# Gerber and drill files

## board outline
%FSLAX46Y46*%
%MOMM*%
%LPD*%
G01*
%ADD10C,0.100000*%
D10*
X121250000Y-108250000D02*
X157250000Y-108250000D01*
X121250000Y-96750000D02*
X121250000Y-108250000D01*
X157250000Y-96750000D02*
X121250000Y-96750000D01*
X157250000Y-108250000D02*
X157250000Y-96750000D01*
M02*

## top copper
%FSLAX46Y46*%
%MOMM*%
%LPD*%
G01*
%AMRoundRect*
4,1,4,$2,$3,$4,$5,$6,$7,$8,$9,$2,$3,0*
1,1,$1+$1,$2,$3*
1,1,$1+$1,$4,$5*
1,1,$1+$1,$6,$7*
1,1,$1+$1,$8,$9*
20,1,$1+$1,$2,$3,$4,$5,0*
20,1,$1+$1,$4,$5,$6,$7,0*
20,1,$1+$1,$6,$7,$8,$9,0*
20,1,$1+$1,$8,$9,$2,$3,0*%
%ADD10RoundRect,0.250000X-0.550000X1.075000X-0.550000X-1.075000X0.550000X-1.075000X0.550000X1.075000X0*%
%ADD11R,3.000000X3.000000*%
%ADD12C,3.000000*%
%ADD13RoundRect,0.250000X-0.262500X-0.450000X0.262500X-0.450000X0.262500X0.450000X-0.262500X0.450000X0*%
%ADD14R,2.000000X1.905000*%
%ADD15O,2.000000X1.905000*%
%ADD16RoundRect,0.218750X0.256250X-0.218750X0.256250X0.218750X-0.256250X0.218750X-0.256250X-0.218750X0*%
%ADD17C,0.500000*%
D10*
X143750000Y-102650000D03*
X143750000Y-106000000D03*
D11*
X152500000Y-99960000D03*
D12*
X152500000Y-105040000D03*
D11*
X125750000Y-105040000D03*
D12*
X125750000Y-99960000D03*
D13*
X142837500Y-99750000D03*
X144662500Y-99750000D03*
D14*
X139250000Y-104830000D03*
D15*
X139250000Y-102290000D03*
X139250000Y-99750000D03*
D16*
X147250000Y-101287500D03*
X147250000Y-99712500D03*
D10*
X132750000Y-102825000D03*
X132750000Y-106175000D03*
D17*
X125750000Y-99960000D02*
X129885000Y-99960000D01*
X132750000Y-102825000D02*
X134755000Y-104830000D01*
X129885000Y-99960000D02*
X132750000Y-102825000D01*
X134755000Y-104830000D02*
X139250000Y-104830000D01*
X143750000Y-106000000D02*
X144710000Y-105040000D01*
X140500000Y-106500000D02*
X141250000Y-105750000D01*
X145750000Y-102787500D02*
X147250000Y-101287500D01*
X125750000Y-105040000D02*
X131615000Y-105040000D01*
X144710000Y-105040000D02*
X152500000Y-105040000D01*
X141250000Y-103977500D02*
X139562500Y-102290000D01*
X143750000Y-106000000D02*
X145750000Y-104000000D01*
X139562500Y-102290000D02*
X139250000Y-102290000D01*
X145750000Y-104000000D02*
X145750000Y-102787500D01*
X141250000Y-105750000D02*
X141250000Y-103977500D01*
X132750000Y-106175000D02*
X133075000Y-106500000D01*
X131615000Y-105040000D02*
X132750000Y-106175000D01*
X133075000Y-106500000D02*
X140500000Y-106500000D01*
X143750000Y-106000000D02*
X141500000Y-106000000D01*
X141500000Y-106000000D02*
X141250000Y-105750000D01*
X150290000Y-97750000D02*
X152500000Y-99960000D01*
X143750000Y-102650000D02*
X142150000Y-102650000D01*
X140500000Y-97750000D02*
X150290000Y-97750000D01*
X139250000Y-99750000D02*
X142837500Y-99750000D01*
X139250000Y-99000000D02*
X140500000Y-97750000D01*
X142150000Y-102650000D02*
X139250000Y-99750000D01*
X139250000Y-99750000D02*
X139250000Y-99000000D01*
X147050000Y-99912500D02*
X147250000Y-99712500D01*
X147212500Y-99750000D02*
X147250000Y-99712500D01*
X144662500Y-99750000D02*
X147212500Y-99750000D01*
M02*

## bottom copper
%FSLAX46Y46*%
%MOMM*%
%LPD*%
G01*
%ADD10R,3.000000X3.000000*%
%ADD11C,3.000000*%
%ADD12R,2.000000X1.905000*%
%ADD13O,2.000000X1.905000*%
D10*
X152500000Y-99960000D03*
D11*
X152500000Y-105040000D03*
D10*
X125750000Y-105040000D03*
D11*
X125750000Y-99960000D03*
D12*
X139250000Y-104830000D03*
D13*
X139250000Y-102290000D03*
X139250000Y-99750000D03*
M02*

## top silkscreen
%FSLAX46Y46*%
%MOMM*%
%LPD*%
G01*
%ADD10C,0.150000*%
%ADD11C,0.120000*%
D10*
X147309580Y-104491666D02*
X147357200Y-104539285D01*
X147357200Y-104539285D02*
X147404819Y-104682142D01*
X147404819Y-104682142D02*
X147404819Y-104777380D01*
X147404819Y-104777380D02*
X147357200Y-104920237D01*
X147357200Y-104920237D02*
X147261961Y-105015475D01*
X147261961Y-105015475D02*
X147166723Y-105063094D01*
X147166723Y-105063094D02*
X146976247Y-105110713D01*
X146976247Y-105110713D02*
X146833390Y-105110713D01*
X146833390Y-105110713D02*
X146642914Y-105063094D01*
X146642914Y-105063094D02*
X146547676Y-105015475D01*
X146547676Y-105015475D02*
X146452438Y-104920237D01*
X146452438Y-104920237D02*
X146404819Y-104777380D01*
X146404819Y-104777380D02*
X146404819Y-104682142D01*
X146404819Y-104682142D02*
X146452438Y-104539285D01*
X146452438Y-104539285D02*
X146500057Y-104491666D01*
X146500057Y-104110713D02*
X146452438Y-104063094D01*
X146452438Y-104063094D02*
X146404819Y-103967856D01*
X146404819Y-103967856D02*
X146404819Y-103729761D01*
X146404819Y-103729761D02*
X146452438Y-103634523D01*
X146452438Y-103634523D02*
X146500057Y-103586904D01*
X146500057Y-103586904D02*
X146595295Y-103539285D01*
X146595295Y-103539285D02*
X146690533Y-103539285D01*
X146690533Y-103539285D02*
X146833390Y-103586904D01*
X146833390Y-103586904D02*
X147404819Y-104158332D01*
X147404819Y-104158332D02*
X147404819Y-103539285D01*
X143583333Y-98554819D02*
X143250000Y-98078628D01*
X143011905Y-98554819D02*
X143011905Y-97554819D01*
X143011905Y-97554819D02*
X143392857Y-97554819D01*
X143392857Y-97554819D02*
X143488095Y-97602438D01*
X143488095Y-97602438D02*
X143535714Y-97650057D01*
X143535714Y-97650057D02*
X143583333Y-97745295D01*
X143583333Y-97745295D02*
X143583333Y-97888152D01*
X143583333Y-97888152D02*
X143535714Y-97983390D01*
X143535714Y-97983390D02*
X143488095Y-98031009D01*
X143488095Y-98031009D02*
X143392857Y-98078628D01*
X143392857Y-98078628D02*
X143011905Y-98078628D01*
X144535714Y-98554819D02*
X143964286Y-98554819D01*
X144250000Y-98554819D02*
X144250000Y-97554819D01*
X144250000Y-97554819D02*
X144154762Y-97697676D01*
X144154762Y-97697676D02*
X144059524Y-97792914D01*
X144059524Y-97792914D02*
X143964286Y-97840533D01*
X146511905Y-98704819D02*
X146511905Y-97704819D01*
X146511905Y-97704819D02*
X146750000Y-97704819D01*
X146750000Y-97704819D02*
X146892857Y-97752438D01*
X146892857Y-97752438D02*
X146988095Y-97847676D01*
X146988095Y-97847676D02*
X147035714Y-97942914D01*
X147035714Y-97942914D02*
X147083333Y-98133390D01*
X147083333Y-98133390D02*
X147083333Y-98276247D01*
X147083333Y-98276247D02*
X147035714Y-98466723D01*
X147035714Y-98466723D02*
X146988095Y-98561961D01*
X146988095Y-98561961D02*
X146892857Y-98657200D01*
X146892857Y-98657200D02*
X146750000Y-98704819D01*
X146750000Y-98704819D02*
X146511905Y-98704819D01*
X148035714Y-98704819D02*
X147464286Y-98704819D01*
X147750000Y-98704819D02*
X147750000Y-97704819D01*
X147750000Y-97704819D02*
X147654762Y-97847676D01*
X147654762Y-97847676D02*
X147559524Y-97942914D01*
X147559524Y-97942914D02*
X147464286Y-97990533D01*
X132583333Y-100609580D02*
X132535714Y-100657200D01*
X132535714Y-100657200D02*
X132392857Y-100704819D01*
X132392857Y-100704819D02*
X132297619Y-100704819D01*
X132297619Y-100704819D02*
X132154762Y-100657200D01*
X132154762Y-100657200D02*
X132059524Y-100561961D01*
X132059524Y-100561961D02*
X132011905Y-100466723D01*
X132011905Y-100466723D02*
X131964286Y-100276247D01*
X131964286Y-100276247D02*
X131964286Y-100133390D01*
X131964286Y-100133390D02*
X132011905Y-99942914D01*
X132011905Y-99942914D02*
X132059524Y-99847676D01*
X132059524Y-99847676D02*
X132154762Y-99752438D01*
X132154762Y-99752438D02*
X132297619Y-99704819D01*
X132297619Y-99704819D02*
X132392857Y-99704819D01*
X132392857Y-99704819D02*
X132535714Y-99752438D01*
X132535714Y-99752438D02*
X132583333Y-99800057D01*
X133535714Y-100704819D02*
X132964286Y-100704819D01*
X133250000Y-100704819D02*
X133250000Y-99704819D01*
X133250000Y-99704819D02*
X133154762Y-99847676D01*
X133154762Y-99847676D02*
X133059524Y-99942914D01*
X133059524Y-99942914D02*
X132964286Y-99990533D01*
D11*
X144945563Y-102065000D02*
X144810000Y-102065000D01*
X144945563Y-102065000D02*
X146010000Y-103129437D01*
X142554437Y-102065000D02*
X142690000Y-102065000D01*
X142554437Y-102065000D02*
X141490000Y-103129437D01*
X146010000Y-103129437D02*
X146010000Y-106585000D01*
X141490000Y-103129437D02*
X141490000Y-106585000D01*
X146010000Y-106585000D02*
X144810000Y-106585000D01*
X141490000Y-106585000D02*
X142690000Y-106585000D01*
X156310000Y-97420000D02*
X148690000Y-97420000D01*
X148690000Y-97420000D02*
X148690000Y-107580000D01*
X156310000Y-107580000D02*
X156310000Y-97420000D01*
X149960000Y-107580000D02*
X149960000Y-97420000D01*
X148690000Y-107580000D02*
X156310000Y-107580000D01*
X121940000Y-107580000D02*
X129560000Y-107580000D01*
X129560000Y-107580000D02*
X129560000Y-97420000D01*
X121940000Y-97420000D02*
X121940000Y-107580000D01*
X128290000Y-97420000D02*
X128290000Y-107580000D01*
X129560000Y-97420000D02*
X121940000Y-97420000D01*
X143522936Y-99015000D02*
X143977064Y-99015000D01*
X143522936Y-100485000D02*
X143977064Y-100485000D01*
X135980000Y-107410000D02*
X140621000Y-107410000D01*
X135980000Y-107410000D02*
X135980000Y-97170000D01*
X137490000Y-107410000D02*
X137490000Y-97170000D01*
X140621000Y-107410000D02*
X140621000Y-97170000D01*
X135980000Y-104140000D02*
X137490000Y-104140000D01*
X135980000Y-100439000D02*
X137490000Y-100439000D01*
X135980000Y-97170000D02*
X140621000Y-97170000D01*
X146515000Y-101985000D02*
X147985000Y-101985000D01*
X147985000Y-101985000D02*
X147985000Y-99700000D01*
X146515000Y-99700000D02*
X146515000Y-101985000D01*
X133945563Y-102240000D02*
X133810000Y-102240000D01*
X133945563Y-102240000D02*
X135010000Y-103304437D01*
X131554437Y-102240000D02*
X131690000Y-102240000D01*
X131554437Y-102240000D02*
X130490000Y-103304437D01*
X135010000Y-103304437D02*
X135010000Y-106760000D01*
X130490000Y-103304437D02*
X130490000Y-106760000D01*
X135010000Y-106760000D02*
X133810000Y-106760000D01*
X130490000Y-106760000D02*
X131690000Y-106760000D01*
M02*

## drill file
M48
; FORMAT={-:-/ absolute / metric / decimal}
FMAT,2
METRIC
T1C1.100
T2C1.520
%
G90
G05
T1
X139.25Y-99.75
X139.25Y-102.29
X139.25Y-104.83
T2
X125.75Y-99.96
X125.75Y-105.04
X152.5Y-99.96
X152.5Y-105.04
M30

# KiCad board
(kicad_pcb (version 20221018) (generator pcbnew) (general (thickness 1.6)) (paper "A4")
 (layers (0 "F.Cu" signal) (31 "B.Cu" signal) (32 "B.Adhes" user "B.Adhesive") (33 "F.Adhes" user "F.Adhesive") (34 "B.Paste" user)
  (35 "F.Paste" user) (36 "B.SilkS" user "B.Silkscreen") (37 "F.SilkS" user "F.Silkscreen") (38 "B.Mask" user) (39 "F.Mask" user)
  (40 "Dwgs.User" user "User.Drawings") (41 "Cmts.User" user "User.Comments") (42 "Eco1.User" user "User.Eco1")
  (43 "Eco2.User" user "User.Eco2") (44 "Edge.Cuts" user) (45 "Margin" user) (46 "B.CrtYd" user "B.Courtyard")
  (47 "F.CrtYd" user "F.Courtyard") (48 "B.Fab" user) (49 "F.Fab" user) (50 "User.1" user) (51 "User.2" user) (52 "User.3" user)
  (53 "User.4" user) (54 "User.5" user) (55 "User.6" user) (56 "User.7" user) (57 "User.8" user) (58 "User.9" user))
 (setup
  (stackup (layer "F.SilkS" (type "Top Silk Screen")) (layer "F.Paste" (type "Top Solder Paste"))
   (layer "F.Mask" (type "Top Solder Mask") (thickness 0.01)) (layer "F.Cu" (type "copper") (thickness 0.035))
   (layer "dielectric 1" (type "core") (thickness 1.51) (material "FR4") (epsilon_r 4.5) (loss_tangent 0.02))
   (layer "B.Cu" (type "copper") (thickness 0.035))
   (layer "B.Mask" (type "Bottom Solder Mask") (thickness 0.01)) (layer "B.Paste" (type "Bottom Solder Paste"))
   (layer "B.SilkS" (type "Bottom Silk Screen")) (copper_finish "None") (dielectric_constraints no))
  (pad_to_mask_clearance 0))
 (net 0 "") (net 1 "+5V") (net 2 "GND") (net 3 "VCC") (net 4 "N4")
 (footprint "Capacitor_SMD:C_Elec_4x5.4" (layer "F.Cu") (at 143.75 104.325 -90)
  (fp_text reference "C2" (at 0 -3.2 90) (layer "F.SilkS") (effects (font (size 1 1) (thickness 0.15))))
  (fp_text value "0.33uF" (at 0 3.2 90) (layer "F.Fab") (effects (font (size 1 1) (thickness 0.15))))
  (fp_line (start -2.26 -1.195563) (end -2.26 -1.06) (stroke (width 0.12) (type solid)) (layer "F.SilkS"))
  (fp_line (start -2.26 -1.195563) (end -1.195563 -2.26) (stroke (width 0.12) (type solid)) (layer "F.SilkS"))
  (fp_line (start -2.26 1.195563) (end -2.26 1.06) (stroke (width 0.12) (type solid)) (layer "F.SilkS"))
  (fp_line (start -2.26 1.195563) (end -1.195563 2.26) (stroke (width 0.12) (type solid)) (layer "F.SilkS"))
  (fp_line (start -1.195563 -2.26) (end 2.26 -2.26) (stroke (width 0.12) (type solid)) (layer "F.SilkS"))
  (fp_line (start -1.195563 2.26) (end 2.26 2.26) (stroke (width 0.12) (type solid)) (layer "F.SilkS"))
  (fp_line (start 2.26 -2.26) (end 2.26 -1.06) (stroke (width 0.12) (type solid)) (layer "F.SilkS"))
  (fp_line (start 2.26 2.26) (end 2.26 1.06) (stroke (width 0.12) (type solid)) (layer "F.SilkS"))
  (pad "1" smd roundrect (at -1.675 0 270) (size 2.65 1.6) (layers "F.Cu" "F.Paste" "F.Mask") (roundrect_rratio 0.15625) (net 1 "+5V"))
  (pad "2" smd roundrect (at 1.675 0 270) (size 2.65 1.6) (layers "F.Cu" "F.Paste" "F.Mask") (roundrect_rratio 0.15625) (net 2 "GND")))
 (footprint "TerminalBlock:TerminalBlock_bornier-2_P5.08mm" (layer "F.Cu") (at 152.5 99.96 -90)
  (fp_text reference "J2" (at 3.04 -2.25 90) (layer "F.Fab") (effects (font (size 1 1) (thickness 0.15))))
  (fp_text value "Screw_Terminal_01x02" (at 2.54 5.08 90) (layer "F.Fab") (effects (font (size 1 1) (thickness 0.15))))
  (fp_line (start -2.54 -3.81) (end -2.54 3.81) (stroke (width 0.12) (type solid)) (layer "F.SilkS"))
  (fp_line (start -2.54 3.81) (end 7.62 3.81) (stroke (width 0.12) (type solid)) (layer "F.SilkS"))
  (fp_line (start 7.62 -3.81) (end -2.54 -3.81) (stroke (width 0.12) (type solid)) (layer "F.SilkS"))
  (fp_line (start 7.62 2.54) (end -2.54 2.54) (stroke (width 0.12) (type solid)) (layer "F.SilkS"))
  (fp_line (start 7.62 3.81) (end 7.62 -3.81) (stroke (width 0.12) (type solid)) (layer "F.SilkS"))
  (pad "1" thru_hole rect (at 0 0 270) (size 3 3) (drill 1.52) (layers "*.Cu" "*.Mask") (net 1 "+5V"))
  (pad "2" thru_hole circle (at 5.08 0 270) (size 3 3) (drill 1.52) (layers "*.Cu" "*.Mask") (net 2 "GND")))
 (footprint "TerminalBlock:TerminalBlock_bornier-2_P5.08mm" (layer "F.Cu") (at 125.75 105.04 90)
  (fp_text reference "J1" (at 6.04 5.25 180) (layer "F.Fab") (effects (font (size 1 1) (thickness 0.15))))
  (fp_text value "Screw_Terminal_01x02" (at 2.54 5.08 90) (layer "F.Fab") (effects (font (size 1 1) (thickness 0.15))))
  (fp_line (start -2.54 -3.81) (end -2.54 3.81) (stroke (width 0.12) (type solid)) (layer "F.SilkS"))
  (fp_line (start -2.54 3.81) (end 7.62 3.81) (stroke (width 0.12) (type solid)) (layer "F.SilkS"))
  (fp_line (start 7.62 -3.81) (end -2.54 -3.81) (stroke (width 0.12) (type solid)) (layer "F.SilkS"))
  (fp_line (start 7.62 2.54) (end -2.54 2.54) (stroke (width 0.12) (type solid)) (layer "F.SilkS"))
  (fp_line (start 7.62 3.81) (end 7.62 -3.81) (stroke (width 0.12) (type solid)) (layer "F.SilkS"))
  (pad "1" thru_hole rect (at 0 0 90) (size 3 3) (drill 1.52) (layers "*.Cu" "*.Mask") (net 2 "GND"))
  (pad "2" thru_hole circle (at 5.08 0 90) (size 3 3) (drill 1.52) (layers "*.Cu" "*.Mask") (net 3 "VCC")))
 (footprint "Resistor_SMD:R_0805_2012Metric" (layer "F.Cu") (at 143.75 99.75)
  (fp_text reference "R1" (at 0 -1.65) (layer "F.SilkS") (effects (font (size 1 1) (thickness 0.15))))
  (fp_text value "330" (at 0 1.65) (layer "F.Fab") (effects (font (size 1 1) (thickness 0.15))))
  (fp_line (start -0.227064 -0.735) (end 0.227064 -0.735) (stroke (width 0.12) (type solid)) (layer "F.SilkS"))
  (fp_line (start -0.227064 0.735) (end 0.227064 0.735) (stroke (width 0.12) (type solid)) (layer "F.SilkS"))
  (pad "1" smd roundrect (at -0.9125 0) (size 1.025 1.4) (layers "F.Cu" "F.Paste" "F.Mask") (roundrect_rratio 0.243902) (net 1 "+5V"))
  (pad "2" smd roundrect (at 0.9125 0) (size 1.025 1.4) (layers "F.Cu" "F.Paste" "F.Mask") (roundrect_rratio 0.243902) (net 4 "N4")))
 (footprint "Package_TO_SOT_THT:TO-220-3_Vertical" (layer "F.Cu") (at 139.25 104.83 90)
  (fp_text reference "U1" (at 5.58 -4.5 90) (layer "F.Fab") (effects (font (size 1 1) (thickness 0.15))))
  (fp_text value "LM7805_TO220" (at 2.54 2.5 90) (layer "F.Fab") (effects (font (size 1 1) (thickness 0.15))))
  (fp_line (start -2.58 -3.27) (end -2.58 1.371) (stroke (width 0.12) (type solid)) (layer "F.SilkS"))
  (fp_line (start -2.58 -3.27) (end 7.66 -3.27) (stroke (width 0.12) (type solid)) (layer "F.SilkS"))
  (fp_line (start -2.58 -1.76) (end 7.66 -1.76) (stroke (width 0.12) (type solid)) (layer "F.SilkS"))
  (fp_line (start -2.58 1.371) (end 7.66 1.371) (stroke (width 0.12) (type solid)) (layer "F.SilkS"))
  (fp_line (start 0.69 -3.27) (end 0.69 -1.76) (stroke (width 0.12) (type solid)) (layer "F.SilkS"))
  (fp_line (start 4.391 -3.27) (end 4.391 -1.76) (stroke (width 0.12) (type solid)) (layer "F.SilkS"))
  (fp_line (start 7.66 -3.27) (end 7.66 1.371) (stroke (width 0.12) (type solid)) (layer "F.SilkS"))
  (pad "1" thru_hole rect (at 0 0 90) (size 1.905 2) (drill 1.1) (layers "*.Cu" "*.Mask") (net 3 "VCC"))
  (pad "2" thru_hole oval (at 2.54 0 90) (size 1.905 2) (drill 1.1) (layers "*.Cu" "*.Mask") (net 2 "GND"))
  (pad "3" thru_hole oval (at 5.08 0 90) (size 1.905 2) (drill 1.1) (layers "*.Cu" "*.Mask") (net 1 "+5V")))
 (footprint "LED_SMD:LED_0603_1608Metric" (layer "F.Cu") (at 147.25 100.5 90)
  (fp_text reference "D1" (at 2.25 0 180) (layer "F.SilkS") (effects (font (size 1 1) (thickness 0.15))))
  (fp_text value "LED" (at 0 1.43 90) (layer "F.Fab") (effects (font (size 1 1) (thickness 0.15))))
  (fp_line (start -1.485 -0.735) (end -1.485 0.735) (stroke (width 0.12) (type solid)) (layer "F.SilkS"))
  (fp_line (start -1.485 0.735) (end 0.8 0.735) (stroke (width 0.12) (type solid)) (layer "F.SilkS"))
  (fp_line (start 0.8 -0.735) (end -1.485 -0.735) (stroke (width 0.12) (type solid)) (layer "F.SilkS"))
  (pad "1" smd roundrect (at -0.7875 0 90) (size 0.875 0.95) (layers "F.Cu" "F.Paste" "F.Mask") (roundrect_rratio 0.25) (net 2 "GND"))
  (pad "2" smd roundrect (at 0.7875 0 90) (size 0.875 0.95) (layers "F.Cu" "F.Paste" "F.Mask") (roundrect_rratio 0.25) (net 4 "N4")))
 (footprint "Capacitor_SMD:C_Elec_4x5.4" (layer "F.Cu") (at 132.75 104.5 -90)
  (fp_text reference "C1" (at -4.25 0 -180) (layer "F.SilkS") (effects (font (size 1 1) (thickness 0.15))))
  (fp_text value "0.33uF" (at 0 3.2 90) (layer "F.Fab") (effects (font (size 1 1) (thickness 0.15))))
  (fp_line (start -2.26 -1.195563) (end -2.26 -1.06) (stroke (width 0.12) (type solid)) (layer "F.SilkS"))
  (fp_line (start -2.26 -1.195563) (end -1.195563 -2.26) (stroke (width 0.12) (type solid)) (layer "F.SilkS"))
  (fp_line (start -2.26 1.195563) (end -2.26 1.06) (stroke (width 0.12) (type solid)) (layer "F.SilkS"))
  (fp_line (start -2.26 1.195563) (end -1.195563 2.26) (stroke (width 0.12) (type solid)) (layer "F.SilkS"))
  (fp_line (start -1.195563 -2.26) (end 2.26 -2.26) (stroke (width 0.12) (type solid)) (layer "F.SilkS"))
  (fp_line (start -1.195563 2.26) (end 2.26 2.26) (stroke (width 0.12) (type solid)) (layer "F.SilkS"))
  (fp_line (start 2.26 -2.26) (end 2.26 -1.06) (stroke (width 0.12) (type solid)) (layer "F.SilkS"))
  (fp_line (start 2.26 2.26) (end 2.26 1.06) (stroke (width 0.12) (type solid)) (layer "F.SilkS"))
  (pad "1" smd roundrect (at -1.675 0 270) (size 2.65 1.6) (layers "F.Cu" "F.Paste" "F.Mask") (roundrect_rratio 0.15625) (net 3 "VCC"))
  (pad "2" smd roundrect (at 1.675 0 270) (size 2.65 1.6) (layers "F.Cu" "F.Paste" "F.Mask") (roundrect_rratio 0.15625) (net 2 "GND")))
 (gr_line (start 121.25 108.25) (end 157.25 108.25) (stroke (width 0.1) (type default)) (layer "Edge.Cuts"))
 (gr_line (start 121.25 96.75) (end 121.25 108.25) (stroke (width 0.1) (type default)) (layer "Edge.Cuts"))
 (gr_line (start 157.25 96.75) (end 121.25 96.75) (stroke (width 0.1) (type default)) (layer "Edge.Cuts"))
 (gr_line (start 157.25 108.25) (end 157.25 96.75) (stroke (width 0.1) (type default)) (layer "Edge.Cuts"))
 (segment (start 125.75 99.96) (end 129.885 99.96) (width 0.5) (layer "F.Cu") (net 3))
 (segment (start 132.75 102.825) (end 134.755 104.83) (width 0.5) (layer "F.Cu") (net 3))
 (segment (start 129.885 99.96) (end 132.75 102.825) (width 0.5) (layer "F.Cu") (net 3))
 (segment (start 134.755 104.83) (end 139.25 104.83) (width 0.5) (layer "F.Cu") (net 3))
 (segment (start 143.75 106) (end 144.71 105.04) (width 0.5) (layer "F.Cu") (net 2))
 (segment (start 140.5 106.5) (end 141.25 105.75) (width 0.5) (layer "F.Cu") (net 2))
 (segment (start 145.75 102.7875) (end 147.25 101.2875) (width 0.5) (layer "F.Cu") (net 2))
 (segment (start 125.75 105.04) (end 131.615 105.04) (width 0.5) (layer "F.Cu") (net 2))
 (segment (start 144.71 105.04) (end 152.5 105.04) (width 0.5) (layer "F.Cu") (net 2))
 (segment (start 141.25 103.9775) (end 139.5625 102.29) (width 0.5) (layer "F.Cu") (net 2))
 (segment (start 143.75 106) (end 145.75 104) (width 0.5) (layer "F.Cu") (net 2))
 (segment (start 139.5625 102.29) (end 139.25 102.29) (width 0.5) (layer "F.Cu") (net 2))
 (segment (start 145.75 104) (end 145.75 102.7875) (width 0.5) (layer "F.Cu") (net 2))
 (segment (start 141.25 105.75) (end 141.25 103.9775) (width 0.5) (layer "F.Cu") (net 2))
 (segment (start 132.75 106.175) (end 133.075 106.5) (width 0.5) (layer "F.Cu") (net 2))
 (segment (start 131.615 105.04) (end 132.75 106.175) (width 0.5) (layer "F.Cu") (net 2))
 (segment (start 133.075 106.5) (end 140.5 106.5) (width 0.5) (layer "F.Cu") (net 2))
 (segment (start 143.75 106) (end 141.5 106) (width 0.5) (layer "F.Cu") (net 2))
 (segment (start 141.5 106) (end 141.25 105.75) (width 0.5) (layer "F.Cu") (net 2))
 (segment (start 150.29 97.75) (end 152.5 99.96) (width 0.5) (layer "F.Cu") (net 1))
 (segment (start 143.75 102.65) (end 142.15 102.65) (width 0.5) (layer "F.Cu") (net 1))
 (segment (start 140.5 97.75) (end 150.29 97.75) (width 0.5) (layer "F.Cu") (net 1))
 (segment (start 139.25 99.75) (end 142.8375 99.75) (width 0.5) (layer "F.Cu") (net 1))
 (segment (start 139.25 99) (end 140.5 97.75) (width 0.5) (layer "F.Cu") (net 1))
 (segment (start 142.15 102.65) (end 139.25 99.75) (width 0.5) (layer "F.Cu") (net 1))
 (segment (start 139.25 99.75) (end 139.25 99) (width 0.5) (layer "F.Cu") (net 1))
 (segment (start 147.05 99.9125) (end 147.25 99.7125) (width 0.5) (layer "F.Cu") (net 4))
 (segment (start 147.2125 99.75) (end 147.25 99.7125) (width 0.5) (layer "F.Cu") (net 4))
 (segment (start 144.6625 99.75) (end 147.2125 99.75) (width 0.5) (layer "F.Cu") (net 4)))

